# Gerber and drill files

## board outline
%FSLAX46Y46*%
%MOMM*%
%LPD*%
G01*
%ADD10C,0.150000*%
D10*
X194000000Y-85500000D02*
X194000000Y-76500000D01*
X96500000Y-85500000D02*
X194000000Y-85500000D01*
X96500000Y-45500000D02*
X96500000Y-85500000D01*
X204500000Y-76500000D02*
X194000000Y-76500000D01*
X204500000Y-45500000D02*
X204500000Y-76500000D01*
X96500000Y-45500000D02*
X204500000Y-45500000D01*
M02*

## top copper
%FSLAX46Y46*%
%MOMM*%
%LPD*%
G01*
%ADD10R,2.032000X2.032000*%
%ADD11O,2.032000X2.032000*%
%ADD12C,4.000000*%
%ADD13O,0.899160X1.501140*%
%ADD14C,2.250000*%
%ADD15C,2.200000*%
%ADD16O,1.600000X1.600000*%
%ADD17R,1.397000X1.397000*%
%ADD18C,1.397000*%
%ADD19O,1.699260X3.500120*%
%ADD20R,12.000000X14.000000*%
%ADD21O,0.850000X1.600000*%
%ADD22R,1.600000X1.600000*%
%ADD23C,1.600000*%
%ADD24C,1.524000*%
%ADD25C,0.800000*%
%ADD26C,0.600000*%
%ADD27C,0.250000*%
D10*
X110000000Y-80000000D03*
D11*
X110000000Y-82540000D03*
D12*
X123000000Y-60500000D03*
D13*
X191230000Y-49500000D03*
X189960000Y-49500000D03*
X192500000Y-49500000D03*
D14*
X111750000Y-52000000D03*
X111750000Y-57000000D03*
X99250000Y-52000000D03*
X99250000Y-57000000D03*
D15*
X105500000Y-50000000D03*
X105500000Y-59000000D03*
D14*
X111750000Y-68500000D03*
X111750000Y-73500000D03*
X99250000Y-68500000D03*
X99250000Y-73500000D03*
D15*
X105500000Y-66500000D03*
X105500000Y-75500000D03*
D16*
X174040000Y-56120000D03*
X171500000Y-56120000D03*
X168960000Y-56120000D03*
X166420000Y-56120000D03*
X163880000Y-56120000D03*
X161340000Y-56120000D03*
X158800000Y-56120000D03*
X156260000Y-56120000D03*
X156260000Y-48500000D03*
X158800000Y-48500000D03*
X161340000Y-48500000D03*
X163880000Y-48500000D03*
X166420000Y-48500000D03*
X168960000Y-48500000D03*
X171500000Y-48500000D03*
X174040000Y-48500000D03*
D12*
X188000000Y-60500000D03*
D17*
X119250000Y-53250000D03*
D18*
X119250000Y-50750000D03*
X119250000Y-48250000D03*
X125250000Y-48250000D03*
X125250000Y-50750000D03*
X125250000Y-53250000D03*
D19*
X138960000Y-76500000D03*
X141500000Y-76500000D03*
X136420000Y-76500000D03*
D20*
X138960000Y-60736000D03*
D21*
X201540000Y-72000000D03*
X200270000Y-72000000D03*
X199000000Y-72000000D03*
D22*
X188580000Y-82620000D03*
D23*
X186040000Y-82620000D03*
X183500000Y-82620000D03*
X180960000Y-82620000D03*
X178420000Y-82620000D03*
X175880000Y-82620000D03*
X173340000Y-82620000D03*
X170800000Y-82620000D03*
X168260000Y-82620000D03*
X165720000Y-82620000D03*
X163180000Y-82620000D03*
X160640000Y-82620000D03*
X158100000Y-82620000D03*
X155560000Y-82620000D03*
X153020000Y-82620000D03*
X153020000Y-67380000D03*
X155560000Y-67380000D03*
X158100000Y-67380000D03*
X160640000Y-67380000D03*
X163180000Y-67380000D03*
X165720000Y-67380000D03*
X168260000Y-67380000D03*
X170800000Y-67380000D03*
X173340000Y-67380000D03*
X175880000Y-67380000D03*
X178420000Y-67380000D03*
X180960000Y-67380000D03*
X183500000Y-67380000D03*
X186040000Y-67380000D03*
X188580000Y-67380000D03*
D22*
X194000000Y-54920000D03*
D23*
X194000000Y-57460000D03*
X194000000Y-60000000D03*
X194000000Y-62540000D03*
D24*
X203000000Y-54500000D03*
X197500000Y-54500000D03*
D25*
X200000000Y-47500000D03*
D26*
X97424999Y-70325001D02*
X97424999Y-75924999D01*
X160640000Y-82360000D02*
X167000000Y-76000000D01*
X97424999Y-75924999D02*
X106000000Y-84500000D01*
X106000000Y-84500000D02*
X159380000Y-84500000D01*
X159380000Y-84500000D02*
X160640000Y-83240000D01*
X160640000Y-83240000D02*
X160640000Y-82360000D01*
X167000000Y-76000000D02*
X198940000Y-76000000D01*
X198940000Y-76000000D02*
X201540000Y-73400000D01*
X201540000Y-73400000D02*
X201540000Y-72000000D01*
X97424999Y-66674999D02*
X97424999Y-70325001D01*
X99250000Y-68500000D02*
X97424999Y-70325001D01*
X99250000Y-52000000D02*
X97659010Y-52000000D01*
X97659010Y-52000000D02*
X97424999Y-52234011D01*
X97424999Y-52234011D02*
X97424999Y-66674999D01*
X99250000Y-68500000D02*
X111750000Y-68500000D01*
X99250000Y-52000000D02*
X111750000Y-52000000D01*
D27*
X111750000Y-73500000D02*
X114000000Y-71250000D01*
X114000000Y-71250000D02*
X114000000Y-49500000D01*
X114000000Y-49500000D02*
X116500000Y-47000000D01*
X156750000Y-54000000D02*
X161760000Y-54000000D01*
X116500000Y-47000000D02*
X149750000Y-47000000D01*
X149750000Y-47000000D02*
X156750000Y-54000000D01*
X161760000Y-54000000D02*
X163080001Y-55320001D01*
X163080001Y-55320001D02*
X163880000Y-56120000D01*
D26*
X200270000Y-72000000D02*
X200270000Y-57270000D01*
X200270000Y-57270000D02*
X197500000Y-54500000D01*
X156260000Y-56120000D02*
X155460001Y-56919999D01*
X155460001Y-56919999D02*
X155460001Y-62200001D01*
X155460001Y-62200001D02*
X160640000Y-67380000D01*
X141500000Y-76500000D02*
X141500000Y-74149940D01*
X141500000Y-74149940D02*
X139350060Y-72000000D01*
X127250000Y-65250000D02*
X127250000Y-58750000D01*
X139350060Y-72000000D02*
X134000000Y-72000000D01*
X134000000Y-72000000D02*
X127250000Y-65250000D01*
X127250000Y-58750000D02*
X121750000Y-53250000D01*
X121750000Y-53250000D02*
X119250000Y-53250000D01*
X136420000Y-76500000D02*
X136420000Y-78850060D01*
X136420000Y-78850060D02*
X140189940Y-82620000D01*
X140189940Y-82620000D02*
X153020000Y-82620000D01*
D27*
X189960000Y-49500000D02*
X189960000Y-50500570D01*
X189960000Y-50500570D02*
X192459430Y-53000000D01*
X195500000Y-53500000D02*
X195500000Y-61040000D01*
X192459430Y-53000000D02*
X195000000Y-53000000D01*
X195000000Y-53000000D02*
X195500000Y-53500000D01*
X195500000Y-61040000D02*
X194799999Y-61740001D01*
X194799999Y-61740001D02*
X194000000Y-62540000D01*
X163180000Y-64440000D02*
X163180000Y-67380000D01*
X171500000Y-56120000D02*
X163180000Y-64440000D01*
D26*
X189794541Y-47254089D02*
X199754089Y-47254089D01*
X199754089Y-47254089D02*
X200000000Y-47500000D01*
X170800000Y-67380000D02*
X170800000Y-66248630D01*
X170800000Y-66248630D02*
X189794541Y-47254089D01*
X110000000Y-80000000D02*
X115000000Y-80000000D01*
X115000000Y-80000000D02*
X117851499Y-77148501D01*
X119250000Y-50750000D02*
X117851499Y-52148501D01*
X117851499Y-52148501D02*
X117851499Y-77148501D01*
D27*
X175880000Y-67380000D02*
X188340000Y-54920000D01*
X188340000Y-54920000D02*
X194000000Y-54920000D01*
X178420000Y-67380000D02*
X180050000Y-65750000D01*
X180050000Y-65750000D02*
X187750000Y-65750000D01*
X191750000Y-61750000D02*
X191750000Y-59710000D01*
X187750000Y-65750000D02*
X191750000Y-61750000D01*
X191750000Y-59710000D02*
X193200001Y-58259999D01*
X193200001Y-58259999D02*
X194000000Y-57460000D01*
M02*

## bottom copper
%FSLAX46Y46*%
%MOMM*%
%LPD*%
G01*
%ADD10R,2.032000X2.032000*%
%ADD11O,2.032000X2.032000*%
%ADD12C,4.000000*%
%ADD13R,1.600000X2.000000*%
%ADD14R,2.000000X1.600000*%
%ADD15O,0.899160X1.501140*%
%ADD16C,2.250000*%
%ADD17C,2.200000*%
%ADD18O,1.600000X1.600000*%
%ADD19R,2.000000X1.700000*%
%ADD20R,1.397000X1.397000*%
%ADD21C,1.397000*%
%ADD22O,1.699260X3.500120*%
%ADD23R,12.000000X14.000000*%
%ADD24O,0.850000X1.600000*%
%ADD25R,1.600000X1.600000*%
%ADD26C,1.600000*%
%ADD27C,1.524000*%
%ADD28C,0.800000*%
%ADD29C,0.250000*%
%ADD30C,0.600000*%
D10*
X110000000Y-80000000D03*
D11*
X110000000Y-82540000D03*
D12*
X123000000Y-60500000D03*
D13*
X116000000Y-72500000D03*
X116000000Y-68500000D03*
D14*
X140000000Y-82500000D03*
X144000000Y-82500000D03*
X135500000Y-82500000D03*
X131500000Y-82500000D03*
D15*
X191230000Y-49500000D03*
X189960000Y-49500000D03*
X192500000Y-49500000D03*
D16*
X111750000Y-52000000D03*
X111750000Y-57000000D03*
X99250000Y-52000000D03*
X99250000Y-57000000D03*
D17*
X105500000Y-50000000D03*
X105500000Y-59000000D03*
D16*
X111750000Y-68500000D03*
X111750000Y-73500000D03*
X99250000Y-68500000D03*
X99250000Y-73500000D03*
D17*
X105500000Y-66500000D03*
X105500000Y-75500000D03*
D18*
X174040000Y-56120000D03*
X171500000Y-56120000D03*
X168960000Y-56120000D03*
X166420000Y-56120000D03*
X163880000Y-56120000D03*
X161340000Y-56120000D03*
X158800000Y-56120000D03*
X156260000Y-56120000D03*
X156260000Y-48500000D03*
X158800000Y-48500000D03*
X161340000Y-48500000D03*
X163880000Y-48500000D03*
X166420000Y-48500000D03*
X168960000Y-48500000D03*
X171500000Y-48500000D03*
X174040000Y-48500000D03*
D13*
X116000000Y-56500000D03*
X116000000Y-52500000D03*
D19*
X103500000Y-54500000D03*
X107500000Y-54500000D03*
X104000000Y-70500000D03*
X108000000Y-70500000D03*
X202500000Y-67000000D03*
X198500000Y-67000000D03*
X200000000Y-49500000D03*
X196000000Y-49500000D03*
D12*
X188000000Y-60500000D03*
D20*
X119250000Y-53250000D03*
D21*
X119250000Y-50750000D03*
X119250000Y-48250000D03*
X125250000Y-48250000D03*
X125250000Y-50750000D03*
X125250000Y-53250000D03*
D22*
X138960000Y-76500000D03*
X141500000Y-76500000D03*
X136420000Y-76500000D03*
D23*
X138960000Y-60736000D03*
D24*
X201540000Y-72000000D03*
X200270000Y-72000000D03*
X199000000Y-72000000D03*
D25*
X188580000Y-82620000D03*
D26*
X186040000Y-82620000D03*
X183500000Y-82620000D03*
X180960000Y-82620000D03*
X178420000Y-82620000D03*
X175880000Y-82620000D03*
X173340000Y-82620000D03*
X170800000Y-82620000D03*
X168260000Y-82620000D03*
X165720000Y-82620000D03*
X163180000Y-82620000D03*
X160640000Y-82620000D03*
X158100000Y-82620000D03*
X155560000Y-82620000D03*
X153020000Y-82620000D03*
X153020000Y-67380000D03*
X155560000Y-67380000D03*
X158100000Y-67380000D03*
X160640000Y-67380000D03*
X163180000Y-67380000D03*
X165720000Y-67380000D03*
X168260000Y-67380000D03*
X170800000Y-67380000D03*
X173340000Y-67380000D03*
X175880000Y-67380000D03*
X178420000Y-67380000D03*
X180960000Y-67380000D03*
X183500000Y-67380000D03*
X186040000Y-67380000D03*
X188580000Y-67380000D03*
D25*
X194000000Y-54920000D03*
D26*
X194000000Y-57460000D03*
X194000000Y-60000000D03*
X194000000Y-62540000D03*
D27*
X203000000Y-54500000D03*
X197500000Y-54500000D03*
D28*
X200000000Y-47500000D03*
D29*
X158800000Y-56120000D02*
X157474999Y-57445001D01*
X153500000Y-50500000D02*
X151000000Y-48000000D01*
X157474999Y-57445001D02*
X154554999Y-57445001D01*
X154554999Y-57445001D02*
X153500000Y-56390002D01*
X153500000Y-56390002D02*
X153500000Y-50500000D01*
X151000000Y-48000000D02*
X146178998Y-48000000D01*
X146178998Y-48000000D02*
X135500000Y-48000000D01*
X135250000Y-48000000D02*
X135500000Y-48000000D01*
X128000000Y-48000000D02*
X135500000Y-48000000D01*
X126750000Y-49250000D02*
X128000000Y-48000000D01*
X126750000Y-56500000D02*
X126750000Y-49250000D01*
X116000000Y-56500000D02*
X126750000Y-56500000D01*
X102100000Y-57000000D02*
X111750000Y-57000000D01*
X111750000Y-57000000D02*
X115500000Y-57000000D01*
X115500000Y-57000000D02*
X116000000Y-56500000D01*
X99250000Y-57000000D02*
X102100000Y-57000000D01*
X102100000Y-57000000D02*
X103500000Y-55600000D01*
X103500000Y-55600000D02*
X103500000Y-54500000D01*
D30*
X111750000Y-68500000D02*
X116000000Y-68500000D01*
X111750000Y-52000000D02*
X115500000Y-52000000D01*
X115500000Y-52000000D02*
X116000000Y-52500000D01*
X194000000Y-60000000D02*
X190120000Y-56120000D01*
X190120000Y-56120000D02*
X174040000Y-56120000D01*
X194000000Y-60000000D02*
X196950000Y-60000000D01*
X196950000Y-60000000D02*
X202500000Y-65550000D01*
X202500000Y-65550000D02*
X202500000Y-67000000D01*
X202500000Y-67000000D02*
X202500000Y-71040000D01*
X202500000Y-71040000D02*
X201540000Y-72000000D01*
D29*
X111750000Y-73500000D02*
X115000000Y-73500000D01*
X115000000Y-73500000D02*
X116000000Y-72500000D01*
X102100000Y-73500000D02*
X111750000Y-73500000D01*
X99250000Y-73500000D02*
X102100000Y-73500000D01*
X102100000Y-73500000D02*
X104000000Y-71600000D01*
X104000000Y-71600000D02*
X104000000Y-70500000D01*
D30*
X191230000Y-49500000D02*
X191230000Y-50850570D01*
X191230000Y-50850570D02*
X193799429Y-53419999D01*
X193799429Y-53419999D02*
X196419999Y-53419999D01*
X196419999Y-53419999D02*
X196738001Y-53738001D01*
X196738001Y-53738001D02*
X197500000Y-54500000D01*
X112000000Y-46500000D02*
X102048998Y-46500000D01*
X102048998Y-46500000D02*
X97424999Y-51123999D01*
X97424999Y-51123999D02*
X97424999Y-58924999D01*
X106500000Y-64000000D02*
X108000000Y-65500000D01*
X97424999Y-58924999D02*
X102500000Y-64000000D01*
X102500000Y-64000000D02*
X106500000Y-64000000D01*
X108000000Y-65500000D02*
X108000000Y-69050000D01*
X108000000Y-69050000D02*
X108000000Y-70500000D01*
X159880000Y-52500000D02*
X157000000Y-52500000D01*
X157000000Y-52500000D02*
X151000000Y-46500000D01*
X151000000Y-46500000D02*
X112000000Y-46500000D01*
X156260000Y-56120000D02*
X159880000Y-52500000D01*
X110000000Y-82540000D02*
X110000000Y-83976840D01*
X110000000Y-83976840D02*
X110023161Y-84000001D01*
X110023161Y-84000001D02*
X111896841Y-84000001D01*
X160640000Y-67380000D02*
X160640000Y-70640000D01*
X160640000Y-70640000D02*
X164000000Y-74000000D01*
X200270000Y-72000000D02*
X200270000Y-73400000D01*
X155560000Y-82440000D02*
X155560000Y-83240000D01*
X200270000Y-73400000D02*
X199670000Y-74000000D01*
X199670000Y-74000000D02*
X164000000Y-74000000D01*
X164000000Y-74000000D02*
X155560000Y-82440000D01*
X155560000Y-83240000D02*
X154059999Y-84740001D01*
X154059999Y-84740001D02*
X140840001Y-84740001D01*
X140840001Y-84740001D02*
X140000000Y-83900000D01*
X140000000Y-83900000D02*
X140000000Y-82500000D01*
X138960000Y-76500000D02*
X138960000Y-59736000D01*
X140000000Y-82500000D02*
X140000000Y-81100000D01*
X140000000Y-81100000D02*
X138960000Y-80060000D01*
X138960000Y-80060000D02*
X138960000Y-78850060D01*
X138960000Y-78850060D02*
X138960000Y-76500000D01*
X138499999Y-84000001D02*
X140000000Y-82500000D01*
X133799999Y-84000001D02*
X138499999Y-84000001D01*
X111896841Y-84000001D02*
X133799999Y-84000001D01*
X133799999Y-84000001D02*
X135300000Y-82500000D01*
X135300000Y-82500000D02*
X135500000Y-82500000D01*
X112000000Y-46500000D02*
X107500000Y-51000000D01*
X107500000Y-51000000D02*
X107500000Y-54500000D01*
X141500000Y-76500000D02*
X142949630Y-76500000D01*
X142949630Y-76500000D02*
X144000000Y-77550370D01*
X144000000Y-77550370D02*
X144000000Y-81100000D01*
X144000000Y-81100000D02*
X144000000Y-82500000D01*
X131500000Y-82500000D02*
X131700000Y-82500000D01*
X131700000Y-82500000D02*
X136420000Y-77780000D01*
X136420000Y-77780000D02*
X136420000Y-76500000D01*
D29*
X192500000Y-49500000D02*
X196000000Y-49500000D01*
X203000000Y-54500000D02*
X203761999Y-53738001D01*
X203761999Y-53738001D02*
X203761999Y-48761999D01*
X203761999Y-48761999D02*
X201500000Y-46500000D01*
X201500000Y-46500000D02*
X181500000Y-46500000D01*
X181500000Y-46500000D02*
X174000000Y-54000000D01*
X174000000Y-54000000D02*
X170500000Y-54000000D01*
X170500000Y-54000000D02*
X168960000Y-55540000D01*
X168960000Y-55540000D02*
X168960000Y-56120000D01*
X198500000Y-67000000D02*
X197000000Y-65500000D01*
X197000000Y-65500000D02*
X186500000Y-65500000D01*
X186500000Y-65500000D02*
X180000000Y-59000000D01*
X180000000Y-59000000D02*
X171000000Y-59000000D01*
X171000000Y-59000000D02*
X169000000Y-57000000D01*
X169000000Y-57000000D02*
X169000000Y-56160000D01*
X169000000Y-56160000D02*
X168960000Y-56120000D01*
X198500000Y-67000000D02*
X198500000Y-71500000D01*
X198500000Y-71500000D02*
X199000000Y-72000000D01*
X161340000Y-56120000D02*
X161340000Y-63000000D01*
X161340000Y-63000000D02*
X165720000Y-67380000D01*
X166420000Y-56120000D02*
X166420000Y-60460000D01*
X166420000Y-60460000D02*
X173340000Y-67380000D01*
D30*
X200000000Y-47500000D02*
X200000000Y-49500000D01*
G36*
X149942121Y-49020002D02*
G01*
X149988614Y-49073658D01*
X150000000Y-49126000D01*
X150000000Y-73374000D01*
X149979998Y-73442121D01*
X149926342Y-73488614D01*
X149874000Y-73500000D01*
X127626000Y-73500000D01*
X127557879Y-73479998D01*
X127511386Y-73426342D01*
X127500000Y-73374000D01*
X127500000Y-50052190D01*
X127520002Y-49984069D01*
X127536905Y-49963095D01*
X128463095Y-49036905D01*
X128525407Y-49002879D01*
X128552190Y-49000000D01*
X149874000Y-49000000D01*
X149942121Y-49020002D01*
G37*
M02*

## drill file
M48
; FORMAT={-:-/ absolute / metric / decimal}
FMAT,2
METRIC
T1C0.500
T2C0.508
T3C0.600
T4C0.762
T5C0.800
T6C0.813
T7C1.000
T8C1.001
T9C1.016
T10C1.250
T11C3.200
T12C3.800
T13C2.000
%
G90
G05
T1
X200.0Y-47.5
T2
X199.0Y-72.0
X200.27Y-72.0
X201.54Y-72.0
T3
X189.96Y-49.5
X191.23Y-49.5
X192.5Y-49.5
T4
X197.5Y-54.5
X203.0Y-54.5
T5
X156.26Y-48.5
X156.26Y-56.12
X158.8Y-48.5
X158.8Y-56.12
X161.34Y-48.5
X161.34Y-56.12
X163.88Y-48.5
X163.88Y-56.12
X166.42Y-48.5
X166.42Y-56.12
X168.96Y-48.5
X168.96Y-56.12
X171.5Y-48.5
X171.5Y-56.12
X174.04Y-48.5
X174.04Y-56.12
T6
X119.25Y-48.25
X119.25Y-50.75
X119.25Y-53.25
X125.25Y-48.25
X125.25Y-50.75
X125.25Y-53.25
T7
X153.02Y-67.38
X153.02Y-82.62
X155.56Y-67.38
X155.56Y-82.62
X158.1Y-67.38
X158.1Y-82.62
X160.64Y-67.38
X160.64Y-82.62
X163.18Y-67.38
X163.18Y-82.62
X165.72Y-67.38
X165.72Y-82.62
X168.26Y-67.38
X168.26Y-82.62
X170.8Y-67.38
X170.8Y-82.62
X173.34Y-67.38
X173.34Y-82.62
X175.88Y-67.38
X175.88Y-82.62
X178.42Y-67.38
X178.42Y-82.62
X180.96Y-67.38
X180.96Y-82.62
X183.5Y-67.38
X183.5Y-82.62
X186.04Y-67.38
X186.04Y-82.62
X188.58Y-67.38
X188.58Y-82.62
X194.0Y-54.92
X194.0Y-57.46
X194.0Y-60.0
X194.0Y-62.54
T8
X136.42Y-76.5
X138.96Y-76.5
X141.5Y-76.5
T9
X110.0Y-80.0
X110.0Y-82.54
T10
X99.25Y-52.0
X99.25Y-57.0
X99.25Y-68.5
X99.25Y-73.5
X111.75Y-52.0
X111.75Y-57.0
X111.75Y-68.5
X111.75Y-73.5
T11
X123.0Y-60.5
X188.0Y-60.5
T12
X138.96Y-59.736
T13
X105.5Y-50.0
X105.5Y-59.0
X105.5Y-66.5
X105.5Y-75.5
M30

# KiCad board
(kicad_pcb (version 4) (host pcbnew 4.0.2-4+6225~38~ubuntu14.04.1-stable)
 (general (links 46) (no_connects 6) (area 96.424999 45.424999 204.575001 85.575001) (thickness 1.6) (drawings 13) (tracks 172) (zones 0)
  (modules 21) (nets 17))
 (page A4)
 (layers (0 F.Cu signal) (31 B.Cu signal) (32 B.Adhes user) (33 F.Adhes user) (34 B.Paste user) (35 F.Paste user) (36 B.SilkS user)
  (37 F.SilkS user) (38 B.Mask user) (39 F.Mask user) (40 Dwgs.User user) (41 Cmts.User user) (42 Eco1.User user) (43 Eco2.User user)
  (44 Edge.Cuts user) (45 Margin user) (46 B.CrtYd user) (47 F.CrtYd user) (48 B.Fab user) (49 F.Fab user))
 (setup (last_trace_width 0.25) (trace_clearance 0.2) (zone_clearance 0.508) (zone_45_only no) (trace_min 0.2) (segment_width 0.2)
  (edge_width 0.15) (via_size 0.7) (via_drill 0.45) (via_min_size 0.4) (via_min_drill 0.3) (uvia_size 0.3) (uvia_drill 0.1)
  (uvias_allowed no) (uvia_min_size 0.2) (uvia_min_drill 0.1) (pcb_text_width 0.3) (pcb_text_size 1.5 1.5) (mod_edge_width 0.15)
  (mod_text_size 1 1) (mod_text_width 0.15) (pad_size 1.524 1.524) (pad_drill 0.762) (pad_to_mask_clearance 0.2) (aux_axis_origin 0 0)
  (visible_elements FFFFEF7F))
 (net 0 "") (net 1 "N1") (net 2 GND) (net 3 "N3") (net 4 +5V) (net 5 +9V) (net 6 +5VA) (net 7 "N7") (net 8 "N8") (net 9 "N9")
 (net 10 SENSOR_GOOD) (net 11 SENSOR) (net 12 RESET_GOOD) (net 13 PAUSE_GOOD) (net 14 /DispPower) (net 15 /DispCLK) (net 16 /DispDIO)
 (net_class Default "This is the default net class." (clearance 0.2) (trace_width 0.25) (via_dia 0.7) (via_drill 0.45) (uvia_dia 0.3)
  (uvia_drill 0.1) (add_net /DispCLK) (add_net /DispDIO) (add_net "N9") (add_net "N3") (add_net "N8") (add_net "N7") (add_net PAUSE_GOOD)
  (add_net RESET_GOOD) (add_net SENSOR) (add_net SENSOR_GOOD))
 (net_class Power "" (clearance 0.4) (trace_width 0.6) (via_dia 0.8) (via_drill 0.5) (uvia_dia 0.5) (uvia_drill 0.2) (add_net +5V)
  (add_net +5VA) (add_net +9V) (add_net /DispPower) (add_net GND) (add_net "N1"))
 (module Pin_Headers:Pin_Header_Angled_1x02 (layer B.Cu) (at 110 80 180)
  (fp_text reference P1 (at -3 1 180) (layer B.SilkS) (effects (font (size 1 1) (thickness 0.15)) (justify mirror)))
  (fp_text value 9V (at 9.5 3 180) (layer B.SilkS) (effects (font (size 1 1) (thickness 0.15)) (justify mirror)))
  (pad 1 thru_hole rect (at 0 0 180) (size 2.032 2.032) (drill 1.016) (layers *.Cu *.Mask B.SilkS) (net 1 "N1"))
  (pad 2 thru_hole oval (at 0 -2.54 180) (size 2.032 2.032) (drill 1.016) (layers *.Cu *.Mask B.SilkS) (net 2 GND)))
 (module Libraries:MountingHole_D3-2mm (layer F.Cu) (at 123 60.5)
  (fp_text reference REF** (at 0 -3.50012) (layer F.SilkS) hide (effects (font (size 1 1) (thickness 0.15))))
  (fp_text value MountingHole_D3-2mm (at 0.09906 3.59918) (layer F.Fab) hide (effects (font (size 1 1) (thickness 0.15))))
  (pad 1 thru_hole circle (at 0 0) (size 4 4) (drill 3.2) (layers *.Cu)))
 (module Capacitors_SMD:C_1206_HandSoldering (layer B.Cu) (at 116 70.5 90)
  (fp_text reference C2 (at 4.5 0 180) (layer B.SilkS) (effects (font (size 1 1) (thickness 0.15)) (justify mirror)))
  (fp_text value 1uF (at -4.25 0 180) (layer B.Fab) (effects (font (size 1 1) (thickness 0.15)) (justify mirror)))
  (pad 1 smd rect (at -2 0 90) (size 2 1.6) (layers B.Cu B.Paste B.Mask) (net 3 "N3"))
  (pad 2 smd rect (at 2 0 90) (size 2 1.6) (layers B.Cu B.Paste B.Mask) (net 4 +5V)))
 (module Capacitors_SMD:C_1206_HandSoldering (layer B.Cu) (at 142 82.5)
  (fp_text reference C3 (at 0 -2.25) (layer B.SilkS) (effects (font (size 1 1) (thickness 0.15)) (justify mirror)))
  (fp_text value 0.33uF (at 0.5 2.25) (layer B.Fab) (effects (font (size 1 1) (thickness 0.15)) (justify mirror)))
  (pad 1 smd rect (at -2 0) (size 2 1.6) (layers B.Cu B.Paste B.Mask) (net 2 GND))
  (pad 2 smd rect (at 2 0) (size 2 1.6) (layers B.Cu B.Paste B.Mask) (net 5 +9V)))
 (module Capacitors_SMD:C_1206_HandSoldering (layer B.Cu) (at 133.5 82.5 180)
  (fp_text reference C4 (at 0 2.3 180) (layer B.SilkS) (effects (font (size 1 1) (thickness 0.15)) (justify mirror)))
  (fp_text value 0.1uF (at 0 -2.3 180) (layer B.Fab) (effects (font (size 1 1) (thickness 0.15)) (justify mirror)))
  (pad 1 smd rect (at -2 0 180) (size 2 1.6) (layers B.Cu B.Paste B.Mask) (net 2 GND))
  (pad 2 smd rect (at 2 0 180) (size 2 1.6) (layers B.Cu B.Paste B.Mask) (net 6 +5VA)))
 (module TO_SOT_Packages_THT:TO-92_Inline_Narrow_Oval (layer B.Cu) (at 192.5 49.5 180)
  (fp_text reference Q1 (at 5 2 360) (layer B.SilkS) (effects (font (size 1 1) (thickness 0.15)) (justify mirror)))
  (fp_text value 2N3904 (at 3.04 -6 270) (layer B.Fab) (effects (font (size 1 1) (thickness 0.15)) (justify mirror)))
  (pad 2 thru_hole oval (at 1.27 0) (size 0.89916 1.50114) (drill 0.6) (layers *.Cu *.Mask B.SilkS) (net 2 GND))
  (pad 3 thru_hole oval (at 2.54 0) (size 0.89916 1.50114) (drill 0.6) (layers *.Cu *.Mask B.SilkS) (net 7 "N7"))
  (pad 1 thru_hole oval (at 0 0) (size 0.89916 1.50114) (drill 0.6) (layers *.Cu *.Mask B.SilkS) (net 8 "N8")))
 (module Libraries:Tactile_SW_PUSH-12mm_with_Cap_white (layer F.Cu) (at 105.5 54.5)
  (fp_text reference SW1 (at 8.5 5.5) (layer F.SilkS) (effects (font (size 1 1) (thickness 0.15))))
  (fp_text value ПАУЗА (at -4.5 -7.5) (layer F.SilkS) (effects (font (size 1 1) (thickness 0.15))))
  (pad 1 thru_hole circle (at 6.25 -2.5) (size 2.25 2.25) (drill 1.25) (layers *.Cu *.Mask F.SilkS) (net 4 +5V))
  (pad 2 thru_hole circle (at 6.25 2.5) (size 2.25 2.25) (drill 1.25) (layers *.Cu *.Mask F.SilkS) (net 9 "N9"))
  (pad 1 thru_hole circle (at -6.25 -2.5) (size 2.25 2.25) (drill 1.25) (layers *.Cu *.Mask F.SilkS) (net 4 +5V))
  (pad 2 thru_hole circle (at -6.25 2.5) (size 2.25 2.25) (drill 1.25) (layers *.Cu *.Mask F.SilkS) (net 9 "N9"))
  (pad "" np_thru_hole circle (at 0 -4.5) (size 2.2 2.2) (drill 2) (layers *.Cu *.Mask F.SilkS))
  (pad "" np_thru_hole circle (at 0 4.5) (size 2.2 2.2) (drill 2) (layers *.Cu *.Mask F.SilkS)))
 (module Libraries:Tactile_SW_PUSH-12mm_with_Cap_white (layer F.Cu) (at 105.5 71)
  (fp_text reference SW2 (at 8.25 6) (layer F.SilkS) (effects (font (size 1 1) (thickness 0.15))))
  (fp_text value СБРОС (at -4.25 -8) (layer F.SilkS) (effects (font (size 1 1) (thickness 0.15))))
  (pad 1 thru_hole circle (at 6.25 -2.5) (size 2.25 2.25) (drill 1.25) (layers *.Cu *.Mask F.SilkS) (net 4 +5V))
  (pad 2 thru_hole circle (at 6.25 2.5) (size 2.25 2.25) (drill 1.25) (layers *.Cu *.Mask F.SilkS) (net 3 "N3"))
  (pad 1 thru_hole circle (at -6.25 -2.5) (size 2.25 2.25) (drill 1.25) (layers *.Cu *.Mask F.SilkS) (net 4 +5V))
  (pad 2 thru_hole circle (at -6.25 2.5) (size 2.25 2.25) (drill 1.25) (layers *.Cu *.Mask F.SilkS) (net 3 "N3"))
  (pad "" np_thru_hole circle (at 0 -4.5) (size 2.2 2.2) (drill 2) (layers *.Cu *.Mask F.SilkS))
  (pad "" np_thru_hole circle (at 0 4.5) (size 2.2 2.2) (drill 2) (layers *.Cu *.Mask F.SilkS)))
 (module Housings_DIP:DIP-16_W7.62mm (layer B.Cu) (at 174.04 56.12 90)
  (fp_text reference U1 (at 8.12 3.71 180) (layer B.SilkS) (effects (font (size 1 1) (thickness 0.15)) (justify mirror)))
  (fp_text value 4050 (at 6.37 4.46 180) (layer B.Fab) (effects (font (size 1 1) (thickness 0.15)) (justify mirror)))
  (pad 1 thru_hole oval (at 0 0 90) (size 1.6 1.6) (drill 0.8) (layers *.Cu *.Mask B.SilkS) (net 4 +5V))
  (pad 2 thru_hole oval (at 0 -2.54 90) (size 1.6 1.6) (drill 0.8) (layers *.Cu *.Mask B.SilkS) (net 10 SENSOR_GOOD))
  (pad 3 thru_hole oval (at 0 -5.08 90) (size 1.6 1.6) (drill 0.8) (layers *.Cu *.Mask B.SilkS) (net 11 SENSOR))
  (pad 4 thru_hole oval (at 0 -7.62 90) (size 1.6 1.6) (drill 0.8) (layers *.Cu *.Mask B.SilkS) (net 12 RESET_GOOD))
  (pad 5 thru_hole oval (at 0 -10.16 90) (size 1.6 1.6) (drill 0.8) (layers *.Cu *.Mask B.SilkS) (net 3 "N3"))
  (pad 6 thru_hole oval (at 0 -12.7 90) (size 1.6 1.6) (drill 0.8) (layers *.Cu *.Mask B.SilkS) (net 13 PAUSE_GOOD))
  (pad 7 thru_hole oval (at 0 -15.24 90) (size 1.6 1.6) (drill 0.8) (layers *.Cu *.Mask B.SilkS) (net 9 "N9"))
  (pad 8 thru_hole oval (at 0 -17.78 90) (size 1.6 1.6) (drill 0.8) (layers *.Cu *.Mask B.SilkS) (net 2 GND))
  (pad 9 thru_hole oval (at 7.62 -17.78 90) (size 1.6 1.6) (drill 0.8) (layers *.Cu *.Mask B.SilkS))
  (pad 10 thru_hole oval (at 7.62 -15.24 90) (size 1.6 1.6) (drill 0.8) (layers *.Cu *.Mask B.SilkS))
  (pad 11 thru_hole oval (at 7.62 -12.7 90) (size 1.6 1.6) (drill 0.8) (layers *.Cu *.Mask B.SilkS))
  (pad 12 thru_hole oval (at 7.62 -10.16 90) (size 1.6 1.6) (drill 0.8) (layers *.Cu *.Mask B.SilkS))
  (pad 13 thru_hole oval (at 7.62 -7.62 90) (size 1.6 1.6) (drill 0.8) (layers *.Cu *.Mask B.SilkS))
  (pad 14 thru_hole oval (at 7.62 -5.08 90) (size 1.6 1.6) (drill 0.8) (layers *.Cu *.Mask B.SilkS))
  (pad 15 thru_hole oval (at 7.62 -2.54 90) (size 1.6 1.6) (drill 0.8) (layers *.Cu *.Mask B.SilkS))
  (pad 16 thru_hole oval (at 7.62 0 90) (size 1.6 1.6) (drill 0.8) (layers *.Cu *.Mask B.SilkS)))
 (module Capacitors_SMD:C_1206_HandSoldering (layer B.Cu) (at 116 54.5 90)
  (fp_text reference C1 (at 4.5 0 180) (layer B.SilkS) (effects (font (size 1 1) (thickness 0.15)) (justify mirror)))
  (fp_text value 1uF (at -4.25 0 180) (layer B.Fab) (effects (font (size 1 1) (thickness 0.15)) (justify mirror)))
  (pad 1 smd rect (at -2 0 90) (size 2 1.6) (layers B.Cu B.Paste B.Mask) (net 9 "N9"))
  (pad 2 smd rect (at 2 0 90) (size 2 1.6) (layers B.Cu B.Paste B.Mask) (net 4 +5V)))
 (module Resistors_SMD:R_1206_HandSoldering (layer B.Cu) (at 105.5 54.5)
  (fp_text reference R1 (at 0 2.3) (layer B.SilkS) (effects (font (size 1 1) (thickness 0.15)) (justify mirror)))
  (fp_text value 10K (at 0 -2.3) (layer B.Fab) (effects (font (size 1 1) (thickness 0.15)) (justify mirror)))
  (pad 1 smd rect (at -2 0) (size 2 1.7) (layers B.Cu B.Paste B.Mask) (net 9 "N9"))
  (pad 2 smd rect (at 2 0) (size 2 1.7) (layers B.Cu B.Paste B.Mask) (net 2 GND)))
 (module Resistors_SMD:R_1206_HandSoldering (layer B.Cu) (at 106 70.5)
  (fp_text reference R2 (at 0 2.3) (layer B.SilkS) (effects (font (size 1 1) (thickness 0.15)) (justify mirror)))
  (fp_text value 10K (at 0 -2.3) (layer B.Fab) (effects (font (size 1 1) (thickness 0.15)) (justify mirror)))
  (pad 1 smd rect (at -2 0) (size 2 1.7) (layers B.Cu B.Paste B.Mask) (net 3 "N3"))
  (pad 2 smd rect (at 2 0) (size 2 1.7) (layers B.Cu B.Paste B.Mask) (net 2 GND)))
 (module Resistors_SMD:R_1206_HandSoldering (layer B.Cu) (at 200.5 67 180)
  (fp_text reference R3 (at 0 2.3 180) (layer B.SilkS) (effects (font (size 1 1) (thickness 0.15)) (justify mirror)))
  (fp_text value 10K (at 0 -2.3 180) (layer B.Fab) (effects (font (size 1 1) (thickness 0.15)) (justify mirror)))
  (pad 1 smd rect (at -2 0 180) (size 2 1.7) (layers B.Cu B.Paste B.Mask) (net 4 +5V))
  (pad 2 smd rect (at 2 0 180) (size 2 1.7) (layers B.Cu B.Paste B.Mask) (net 11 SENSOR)))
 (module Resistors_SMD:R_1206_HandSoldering (layer B.Cu) (at 198 49.5 180)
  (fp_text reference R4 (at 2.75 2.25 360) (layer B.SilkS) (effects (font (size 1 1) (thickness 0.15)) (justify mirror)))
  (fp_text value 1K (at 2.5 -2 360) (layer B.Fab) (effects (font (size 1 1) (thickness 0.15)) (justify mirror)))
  (pad 1 smd rect (at -2 0 180) (size 2 1.7) (layers B.Cu B.Paste B.Mask) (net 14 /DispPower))
  (pad 2 smd rect (at 2 0 180) (size 2 1.7) (layers B.Cu B.Paste B.Mask) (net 8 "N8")))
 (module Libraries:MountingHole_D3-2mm (layer F.Cu) (at 188 60.5)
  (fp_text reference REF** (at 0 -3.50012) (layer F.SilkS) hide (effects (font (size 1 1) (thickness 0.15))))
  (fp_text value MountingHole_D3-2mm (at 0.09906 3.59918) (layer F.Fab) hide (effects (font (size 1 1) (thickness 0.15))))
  (pad 1 thru_hole circle (at 0 0) (size 4 4) (drill 3.2) (layers *.Cu)))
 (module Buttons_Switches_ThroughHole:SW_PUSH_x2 (layer B.Cu) (at 119.25 53.25 90)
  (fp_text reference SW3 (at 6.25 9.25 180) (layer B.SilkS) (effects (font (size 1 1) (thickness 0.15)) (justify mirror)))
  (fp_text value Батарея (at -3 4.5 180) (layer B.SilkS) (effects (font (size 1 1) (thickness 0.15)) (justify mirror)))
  (pad 1 thru_hole rect (at 0 0 90) (size 1.397 1.397) (drill 0.8128) (layers *.Cu *.Mask B.SilkS) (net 5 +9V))
  (pad 2 thru_hole circle (at 2.5 0 90) (size 1.397 1.397) (drill 0.8128) (layers *.Cu *.Mask B.SilkS) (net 1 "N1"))
  (pad 3 thru_hole circle (at 5 0 90) (size 1.397 1.397) (drill 0.8128) (layers *.Cu *.Mask B.SilkS))
  (pad 4 thru_hole circle (at 5 6 90) (size 1.397 1.397) (drill 0.8128) (layers *.Cu *.Mask B.SilkS))
  (pad 5 thru_hole circle (at 2.5 6 90) (size 1.397 1.397) (drill 0.8128) (layers *.Cu *.Mask B.SilkS))
  (pad 6 thru_hole circle (at 0 6 90) (size 1.397 1.397) (drill 0.8128) (layers *.Cu *.Mask B.SilkS)))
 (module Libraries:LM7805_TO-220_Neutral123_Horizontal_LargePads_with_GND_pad (layer B.Cu) (at 138.96 76.5 180)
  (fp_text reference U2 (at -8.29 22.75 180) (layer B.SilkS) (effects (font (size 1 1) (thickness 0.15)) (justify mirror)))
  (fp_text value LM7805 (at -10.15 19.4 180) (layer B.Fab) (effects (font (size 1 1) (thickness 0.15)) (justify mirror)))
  (pad 2 thru_hole oval (at 0 0 90) (size 3.50012 1.69926) (drill 1.00076) (layers *.Cu *.Mask B.SilkS) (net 2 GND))
  (pad 1 thru_hole oval (at -2.54 0 90) (size 3.50012 1.69926) (drill 1.00076) (layers *.Cu *.Mask B.SilkS) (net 5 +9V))
  (pad 3 thru_hole oval (at 2.54 0 90) (size 3.50012 1.69926) (drill 1.00076) (layers *.Cu *.Mask B.SilkS) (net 6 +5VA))
  (pad 2 thru_hole rect (at 0 16.764 90) (size 14 12) (drill 3.79984 (offset -1 0)) (layers B.Cu B.SilkS B.Mask) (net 2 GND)))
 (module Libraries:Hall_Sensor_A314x (layer F.Cu) (at 200.27 72 180)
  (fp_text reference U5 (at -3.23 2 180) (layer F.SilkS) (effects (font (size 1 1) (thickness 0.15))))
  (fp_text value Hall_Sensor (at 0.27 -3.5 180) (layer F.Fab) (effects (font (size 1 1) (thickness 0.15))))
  (pad 1 thru_hole oval (at -1.27 0 180) (size 0.85 1.6) (drill 0.508) (layers *.Cu *.Mask F.SilkS) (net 4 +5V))
  (pad 2 thru_hole oval (at 0 0 180) (size 0.85 1.6) (drill 0.508) (layers *.Cu *.Mask F.SilkS) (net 2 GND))
  (pad 3 thru_hole oval (at 1.27 0 180) (size 0.85 1.6) (drill 0.508) (layers *.Cu *.Mask F.SilkS) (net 11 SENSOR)))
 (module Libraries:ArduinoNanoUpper (layer B.Cu) (at 170.8 75 180)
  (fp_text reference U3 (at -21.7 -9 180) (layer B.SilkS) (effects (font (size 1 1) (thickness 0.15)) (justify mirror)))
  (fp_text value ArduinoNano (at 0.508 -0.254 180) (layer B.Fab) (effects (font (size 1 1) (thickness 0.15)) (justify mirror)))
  (pad 1 thru_hole rect (at -17.78 -7.62 180) (size 1.6 1.6) (drill 1) (layers *.Cu *.Mask B.SilkS))
  (pad 2 thru_hole circle (at -15.24 -7.62 180) (size 1.6 1.6) (drill 1) (layers *.Cu *.Mask B.SilkS))
  (pad 3 thru_hole circle (at -12.7 -7.62 180) (size 1.6 1.6) (drill 1) (layers *.Cu *.Mask B.SilkS))
  (pad 4 thru_hole circle (at -10.16 -7.62 180) (size 1.6 1.6) (drill 1) (layers *.Cu *.Mask B.SilkS))
  (pad 5 thru_hole circle (at -7.62 -7.62 180) (size 1.6 1.6) (drill 1) (layers *.Cu *.Mask B.SilkS))
  (pad 6 thru_hole circle (at -5.08 -7.62 180) (size 1.6 1.6) (drill 1) (layers *.Cu *.Mask B.SilkS))
  (pad 7 thru_hole circle (at -2.54 -7.62 180) (size 1.6 1.6) (drill 1) (layers *.Cu *.Mask B.SilkS))
  (pad 8 thru_hole circle (at 0 -7.62 180) (size 1.6 1.6) (drill 1) (layers *.Cu *.Mask B.SilkS))
  (pad 9 thru_hole circle (at 2.54 -7.62 180) (size 1.6 1.6) (drill 1) (layers *.Cu *.Mask B.SilkS))
  (pad 10 thru_hole circle (at 5.08 -7.62 180) (size 1.6 1.6) (drill 1) (layers *.Cu *.Mask B.SilkS))
  (pad 11 thru_hole circle (at 7.62 -7.62 180) (size 1.6 1.6) (drill 1) (layers *.Cu *.Mask B.SilkS))
  (pad 12 thru_hole circle (at 10.16 -7.62 180) (size 1.6 1.6) (drill 1) (layers *.Cu *.Mask B.SilkS) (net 4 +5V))
  (pad 13 thru_hole circle (at 12.7 -7.62 180) (size 1.6 1.6) (drill 1) (layers *.Cu *.Mask B.SilkS))
  (pad 14 thru_hole circle (at 15.24 -7.62 180) (size 1.6 1.6) (drill 1) (layers *.Cu *.Mask B.SilkS) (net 2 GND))
  (pad 15 thru_hole circle (at 17.78 -7.62 180) (size 1.6 1.6) (drill 1) (layers *.Cu *.Mask B.SilkS) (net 6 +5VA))
  (pad 16 thru_hole circle (at 17.78 7.62 180) (size 1.6 1.6) (drill 1) (layers *.Cu *.Mask B.SilkS))
  (pad 17 thru_hole circle (at 15.24 7.62 180) (size 1.6 1.6) (drill 1) (layers *.Cu *.Mask B.SilkS))
  (pad 18 thru_hole circle (at 12.7 7.62 180) (size 1.6 1.6) (drill 1) (layers *.Cu *.Mask B.SilkS))
  (pad 19 thru_hole circle (at 10.16 7.62 180) (size 1.6 1.6) (drill 1) (layers *.Cu *.Mask B.SilkS) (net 2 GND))
  (pad 20 thru_hole circle (at 7.62 7.62 180) (size 1.6 1.6) (drill 1) (layers *.Cu *.Mask B.SilkS) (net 10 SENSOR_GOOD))
  (pad 21 thru_hole circle (at 5.08 7.62 180) (size 1.6 1.6) (drill 1) (layers *.Cu *.Mask B.SilkS) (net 13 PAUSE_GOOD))
  (pad 22 thru_hole circle (at 2.54 7.62 180) (size 1.6 1.6) (drill 1) (layers *.Cu *.Mask B.SilkS))
  (pad 23 thru_hole circle (at 0 7.62 180) (size 1.6 1.6) (drill 1) (layers *.Cu *.Mask B.SilkS) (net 14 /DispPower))
  (pad 24 thru_hole circle (at -2.54 7.62 180) (size 1.6 1.6) (drill 1) (layers *.Cu *.Mask B.SilkS) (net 12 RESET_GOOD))
  (pad 25 thru_hole circle (at -5.08 7.62 180) (size 1.6 1.6) (drill 1) (layers *.Cu *.Mask B.SilkS) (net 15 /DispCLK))
  (pad 26 thru_hole circle (at -7.62 7.62 180) (size 1.6 1.6) (drill 1) (layers *.Cu *.Mask B.SilkS) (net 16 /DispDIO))
  (pad 27 thru_hole circle (at -10.16 7.62 180) (size 1.6 1.6) (drill 1) (layers *.Cu *.Mask B.SilkS))
  (pad 28 thru_hole circle (at -12.7 7.62 180) (size 1.6 1.6) (drill 1) (layers *.Cu *.Mask B.SilkS))
  (pad 29 thru_hole circle (at -15.24 7.62 180) (size 1.6 1.6) (drill 1) (layers *.Cu *.Mask B.SilkS))
  (pad 30 thru_hole circle (at -17.78 7.62 180) (size 1.6 1.6) (drill 1) (layers *.Cu *.Mask B.SilkS)))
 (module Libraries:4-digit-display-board (layer F.Cu) (at 175.54 58.73)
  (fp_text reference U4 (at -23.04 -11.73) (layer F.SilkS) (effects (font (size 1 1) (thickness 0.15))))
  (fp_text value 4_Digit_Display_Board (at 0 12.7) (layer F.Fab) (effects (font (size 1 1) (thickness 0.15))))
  (pad 1 thru_hole rect (at 18.46 -3.81) (size 1.6 1.6) (drill 1) (layers *.Cu *.Mask F.SilkS) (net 15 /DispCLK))
  (pad 2 thru_hole circle (at 18.46 -1.27) (size 1.6 1.6) (drill 1) (layers *.Cu *.Mask F.SilkS) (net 16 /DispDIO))
  (pad 3 thru_hole circle (at 18.46 1.27) (size 1.6 1.6) (drill 1) (layers *.Cu *.Mask F.SilkS) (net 4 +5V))
  (pad 4 thru_hole circle (at 18.46 3.81) (size 1.6 1.6) (drill 1) (layers *.Cu *.Mask F.SilkS) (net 7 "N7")))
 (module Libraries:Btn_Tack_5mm (layer F.Cu) (at 203 54.5 180)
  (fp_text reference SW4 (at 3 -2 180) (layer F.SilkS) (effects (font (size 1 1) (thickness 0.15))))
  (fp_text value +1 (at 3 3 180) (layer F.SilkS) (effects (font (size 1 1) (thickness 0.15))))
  (pad 1 thru_hole circle (at 0 0 180) (size 1.524 1.524) (drill 0.762) (layers *.Cu *.Mask F.SilkS) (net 11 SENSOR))
  (pad 2 thru_hole circle (at 5.5 0 180) (size 1.524 1.524) (drill 0.762) (layers *.Cu *.Mask F.SilkS) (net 2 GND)))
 (gr_line (start 194 85.5) (end 194 76.5) (layer Edge.Cuts) (width 0.15))
 (gr_line (start 96.5 85.5) (end 194 85.5) (layer Edge.Cuts) (width 0.15))
 (gr_line (start 96.5 45.5) (end 96.5 85.5) (layer Edge.Cuts) (width 0.15))
 (gr_line (start 204.5 76.5) (end 194 76.5) (layer Edge.Cuts) (width 0.15))
 (gr_line (start 204.5 45.5) (end 204.5 76.5) (layer Edge.Cuts) (width 0.15))
 (gr_line (start 96.5 45.5) (end 204.5 45.5) (layer Edge.Cuts) (width 0.15))
 (segment (start 158.8 56.12) (end 157.474999 57.445001) (width 0.25) (layer B.Cu) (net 9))
 (segment (start 153.5 50.5) (end 151 48) (width 0.25) (layer B.Cu) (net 9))
 (segment (start 157.474999 57.445001) (end 154.554999 57.445001) (width 0.25) (layer B.Cu) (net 9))
 (segment (start 154.554999 57.445001) (end 153.5 56.390002) (width 0.25) (layer B.Cu) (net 9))
 (segment (start 153.5 56.390002) (end 153.5 50.5) (width 0.25) (layer B.Cu) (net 9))
 (segment (start 151 48) (end 146.178998 48) (width 0.25) (layer B.Cu) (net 9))
 (segment (start 146.178998 48) (end 135.5 48) (width 0.25) (layer B.Cu) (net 9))
 (segment (start 135.25 48) (end 135.5 48) (width 0.25) (layer B.Cu) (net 9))
 (segment (start 128 48) (end 135.5 48) (width 0.25) (layer B.Cu) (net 9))
 (segment (start 126.75 49.25) (end 128 48) (width 0.25) (layer B.Cu) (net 9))
 (segment (start 126.75 56.5) (end 126.75 49.25) (width 0.25) (layer B.Cu) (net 9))
 (segment (start 116 56.5) (end 126.75 56.5) (width 0.25) (layer B.Cu) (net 9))
 (segment (start 102.1 57) (end 111.75 57) (width 0.25) (layer B.Cu) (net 9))
 (segment (start 111.75 57) (end 115.5 57) (width 0.25) (layer B.Cu) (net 9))
 (segment (start 115.5 57) (end 116 56.5) (width 0.25) (layer B.Cu) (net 9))
 (segment (start 99.25 57) (end 102.1 57) (width 0.25) (layer B.Cu) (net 9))
 (segment (start 102.1 57) (end 103.5 55.6) (width 0.25) (layer B.Cu) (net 9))
 (segment (start 103.5 55.6) (end 103.5 54.5) (width 0.25) (layer B.Cu) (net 9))
 (segment (start 97.424999 70.325001) (end 97.424999 75.924999) (width 0.6) (layer F.Cu) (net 4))
 (segment (start 160.64 82.36) (end 167 76) (width 0.6) (layer F.Cu) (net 4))
 (segment (start 97.424999 75.924999) (end 106 84.5) (width 0.6) (layer F.Cu) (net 4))
 (segment (start 106 84.5) (end 159.38 84.5) (width 0.6) (layer F.Cu) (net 4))
 (segment (start 159.38 84.5) (end 160.64 83.24) (width 0.6) (layer F.Cu) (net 4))
 (segment (start 160.64 83.24) (end 160.64 82.36) (width 0.6) (layer F.Cu) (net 4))
 (segment (start 167 76) (end 198.94 76) (width 0.6) (layer F.Cu) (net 4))
 (segment (start 198.94 76) (end 201.54 73.4) (width 0.6) (layer F.Cu) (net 4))
 (segment (start 201.54 73.4) (end 201.54 72) (width 0.6) (layer F.Cu) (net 4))
 (segment (start 97.424999 66.674999) (end 97.424999 70.325001) (width 0.6) (layer F.Cu) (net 4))
 (segment (start 99.25 68.5) (end 97.424999 70.325001) (width 0.6) (layer F.Cu) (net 4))
 (segment (start 99.25 52) (end 97.65901 52) (width 0.6) (layer F.Cu) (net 4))
 (segment (start 97.65901 52) (end 97.424999 52.234011) (width 0.6) (layer F.Cu) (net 4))
 (segment (start 97.424999 52.234011) (end 97.424999 66.674999) (width 0.6) (layer F.Cu) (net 4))
 (segment (start 99.25 68.5) (end 111.75 68.5) (width 0.6) (layer F.Cu) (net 4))
 (segment (start 99.25 52) (end 111.75 52) (width 0.6) (layer F.Cu) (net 4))
 (segment (start 111.75 68.5) (end 116 68.5) (width 0.6) (layer B.Cu) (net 4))
 (segment (start 111.75 52) (end 115.5 52) (width 0.6) (layer B.Cu) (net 4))
 (segment (start 115.5 52) (end 116 52.5) (width 0.6) (layer B.Cu) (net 4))
 (segment (start 194 60) (end 190.12 56.12) (width 0.6) (layer B.Cu) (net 4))
 (segment (start 190.12 56.12) (end 174.04 56.12) (width 0.6) (layer B.Cu) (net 4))
 (segment (start 194 60) (end 196.95 60) (width 0.6) (layer B.Cu) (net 4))
 (segment (start 196.95 60) (end 202.5 65.55) (width 0.6) (layer B.Cu) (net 4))
 (segment (start 202.5 65.55) (end 202.5 67) (width 0.6) (layer B.Cu) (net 4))
 (segment (start 202.5 67) (end 202.5 71.04) (width 0.6) (layer B.Cu) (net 4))
 (segment (start 202.5 71.04) (end 201.54 72) (width 0.6) (layer B.Cu) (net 4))
 (segment (start 111.75 73.5) (end 114 71.25) (width 0.25) (layer F.Cu) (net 3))
 (segment (start 114 71.25) (end 114 49.5) (width 0.25) (layer F.Cu) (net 3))
 (segment (start 114 49.5) (end 116.5 47) (width 0.25) (layer F.Cu) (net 3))
 (segment (start 156.75 54) (end 161.76 54) (width 0.25) (layer F.Cu) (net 3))
 (segment (start 116.5 47) (end 149.75 47) (width 0.25) (layer F.Cu) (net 3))
 (segment (start 149.75 47) (end 156.75 54) (width 0.25) (layer F.Cu) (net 3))
 (segment (start 161.76 54) (end 163.080001 55.320001) (width 0.25) (layer F.Cu) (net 3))
 (segment (start 163.080001 55.320001) (end 163.88 56.12) (width 0.25) (layer F.Cu) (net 3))
 (segment (start 111.75 73.5) (end 115 73.5) (width 0.25) (layer B.Cu) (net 3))
 (segment (start 115 73.5) (end 116 72.5) (width 0.25) (layer B.Cu) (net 3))
 (segment (start 102.1 73.5) (end 111.75 73.5) (width 0.25) (layer B.Cu) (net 3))
 (segment (start 99.25 73.5) (end 102.1 73.5) (width 0.25) (layer B.Cu) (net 3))
 (segment (start 102.1 73.5) (end 104 71.6) (width 0.25) (layer B.Cu) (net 3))
 (segment (start 104 71.6) (end 104 70.5) (width 0.25) (layer B.Cu) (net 3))
 (segment (start 200.27 72) (end 200.27 57.27) (width 0.6) (layer F.Cu) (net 2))
 (segment (start 200.27 57.27) (end 197.5 54.5) (width 0.6) (layer F.Cu) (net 2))
 (segment (start 191.23 49.5) (end 191.23 50.85057) (width 0.6) (layer B.Cu) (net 2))
 (segment (start 191.23 50.85057) (end 193.799429 53.419999) (width 0.6) (layer B.Cu) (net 2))
 (segment (start 193.799429 53.419999) (end 196.419999 53.419999) (width 0.6) (layer B.Cu) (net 2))
 (segment (start 196.419999 53.419999) (end 196.738001 53.738001) (width 0.6) (layer B.Cu) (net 2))
 (segment (start 196.738001 53.738001) (end 197.5 54.5) (width 0.6) (layer B.Cu) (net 2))
 (segment (start 112 46.5) (end 102.048998 46.5) (width 0.6) (layer B.Cu) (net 2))
 (segment (start 102.048998 46.5) (end 97.424999 51.123999) (width 0.6) (layer B.Cu) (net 2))
 (segment (start 97.424999 51.123999) (end 97.424999 58.924999) (width 0.6) (layer B.Cu) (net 2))
 (segment (start 106.5 64) (end 108 65.5) (width 0.6) (layer B.Cu) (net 2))
 (segment (start 97.424999 58.924999) (end 102.5 64) (width 0.6) (layer B.Cu) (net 2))
 (segment (start 102.5 64) (end 106.5 64) (width 0.6) (layer B.Cu) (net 2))
 (segment (start 108 65.5) (end 108 69.05) (width 0.6) (layer B.Cu) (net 2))
 (segment (start 108 69.05) (end 108 70.5) (width 0.6) (layer B.Cu) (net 2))
 (segment (start 159.88 52.5) (end 157 52.5) (width 0.6) (layer B.Cu) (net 2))
 (segment (start 157 52.5) (end 151 46.5) (width 0.6) (layer B.Cu) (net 2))
 (segment (start 151 46.5) (end 112 46.5) (width 0.6) (layer B.Cu) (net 2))
 (segment (start 156.26 56.12) (end 159.88 52.5) (width 0.6) (layer B.Cu) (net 2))
 (segment (start 110 82.54) (end 110 83.97684) (width 0.6) (layer B.Cu) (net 2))
 (segment (start 110 83.97684) (end 110.023161 84.000001) (width 0.6) (layer B.Cu) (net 2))
 (segment (start 110.023161 84.000001) (end 111.896841 84.000001) (width 0.6) (layer B.Cu) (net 2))
 (segment (start 160.64 67.38) (end 160.64 70.64) (width 0.6) (layer B.Cu) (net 2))
 (segment (start 160.64 70.64) (end 164 74) (width 0.6) (layer B.Cu) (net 2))
 (segment (start 156.26 56.12) (end 155.460001 56.919999) (width 0.6) (layer F.Cu) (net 2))
 (segment (start 155.460001 56.919999) (end 155.460001 62.200001) (width 0.6) (layer F.Cu) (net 2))
 (segment (start 155.460001 62.200001) (end 160.64 67.38) (width 0.6) (layer F.Cu) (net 2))
 (segment (start 200.27 72) (end 200.27 73.4) (width 0.6) (layer B.Cu) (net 2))
 (segment (start 155.56 82.44) (end 155.56 83.24) (width 0.6) (layer B.Cu) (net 2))
 (segment (start 200.27 73.4) (end 199.67 74) (width 0.6) (layer B.Cu) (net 2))
 (segment (start 199.67 74) (end 164 74) (width 0.6) (layer B.Cu) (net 2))
 (segment (start 164 74) (end 155.56 82.44) (width 0.6) (layer B.Cu) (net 2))
 (segment (start 155.56 83.24) (end 154.059999 84.740001) (width 0.6) (layer B.Cu) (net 2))
 (segment (start 154.059999 84.740001) (end 140.840001 84.740001) (width 0.6) (layer B.Cu) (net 2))
 (segment (start 140.840001 84.740001) (end 140 83.9) (width 0.6) (layer B.Cu) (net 2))
 (segment (start 140 83.9) (end 140 82.5) (width 0.6) (layer B.Cu) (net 2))
 (segment (start 138.96 76.5) (end 138.96 59.736) (width 0.6) (layer B.Cu) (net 2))
 (segment (start 140 82.5) (end 140 81.1) (width 0.6) (layer B.Cu) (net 2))
 (segment (start 140 81.1) (end 138.96 80.06) (width 0.6) (layer B.Cu) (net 2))
 (segment (start 138.96 80.06) (end 138.96 78.85006) (width 0.6) (layer B.Cu) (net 2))
 (segment (start 138.96 78.85006) (end 138.96 76.5) (width 0.6) (layer B.Cu) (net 2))
 (segment (start 138.499999 84.000001) (end 140 82.5) (width 0.6) (layer B.Cu) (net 2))
 (segment (start 133.799999 84.000001) (end 138.499999 84.000001) (width 0.6) (layer B.Cu) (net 2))
 (segment (start 111.896841 84.000001) (end 133.799999 84.000001) (width 0.6) (layer B.Cu) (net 2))
 (segment (start 133.799999 84.000001) (end 135.3 82.5) (width 0.6) (layer B.Cu) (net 2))
 (segment (start 135.3 82.5) (end 135.5 82.5) (width 0.6) (layer B.Cu) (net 2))
 (segment (start 112 46.5) (end 107.5 51) (width 0.6) (layer B.Cu) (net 2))
 (segment (start 107.5 51) (end 107.5 54.5) (width 0.6) (layer B.Cu) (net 2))
 (segment (start 141.5 76.5) (end 141.5 74.14994) (width 0.6) (layer F.Cu) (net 5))
 (segment (start 141.5 74.14994) (end 139.35006 72) (width 0.6) (layer F.Cu) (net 5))
 (segment (start 127.25 65.25) (end 127.25 58.75) (width 0.6) (layer F.Cu) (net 5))
 (segment (start 139.35006 72) (end 134 72) (width 0.6) (layer F.Cu) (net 5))
 (segment (start 134 72) (end 127.25 65.25) (width 0.6) (layer F.Cu) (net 5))
 (segment (start 127.25 58.75) (end 121.75 53.25) (width 0.6) (layer F.Cu) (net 5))
 (segment (start 121.75 53.25) (end 119.25 53.25) (width 0.6) (layer F.Cu) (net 5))
 (segment (start 141.5 76.5) (end 142.94963 76.5) (width 0.6) (layer B.Cu) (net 5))
 (segment (start 142.94963 76.5) (end 144 77.55037) (width 0.6) (layer B.Cu) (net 5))
 (segment (start 144 77.55037) (end 144 81.1) (width 0.6) (layer B.Cu) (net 5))
 (segment (start 144 81.1) (end 144 82.5) (width 0.6) (layer B.Cu) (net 5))
 (segment (start 136.42 76.5) (end 136.42 78.85006) (width 0.6) (layer F.Cu) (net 6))
 (segment (start 136.42 78.85006) (end 140.18994 82.62) (width 0.6) (layer F.Cu) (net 6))
 (segment (start 140.18994 82.62) (end 153.02 82.62) (width 0.6) (layer F.Cu) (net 6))
 (segment (start 131.5 82.5) (end 131.7 82.5) (width 0.6) (layer B.Cu) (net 6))
 (segment (start 131.7 82.5) (end 136.42 77.78) (width 0.6) (layer B.Cu) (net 6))
 (segment (start 136.42 77.78) (end 136.42 76.5) (width 0.6) (layer B.Cu) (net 6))
 (segment (start 189.96 49.5) (end 189.96 50.50057) (width 0.25) (layer F.Cu) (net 7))
 (segment (start 189.96 50.50057) (end 192.45943 53) (width 0.25) (layer F.Cu) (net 7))
 (segment (start 195.5 53.5) (end 195.5 61.04) (width 0.25) (layer F.Cu) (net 7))
 (segment (start 192.45943 53) (end 195 53) (width 0.25) (layer F.Cu) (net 7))
 (segment (start 195 53) (end 195.5 53.5) (width 0.25) (layer F.Cu) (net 7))
 (segment (start 195.5 61.04) (end 194.799999 61.740001) (width 0.25) (layer F.Cu) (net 7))
 (segment (start 194.799999 61.740001) (end 194 62.54) (width 0.25) (layer F.Cu) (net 7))
 (segment (start 192.5 49.5) (end 196 49.5) (width 0.25) (layer B.Cu) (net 8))
 (segment (start 163.18 64.44) (end 163.18 67.38) (width 0.25) (layer F.Cu) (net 10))
 (segment (start 171.5 56.12) (end 163.18 64.44) (width 0.25) (layer F.Cu) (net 10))
 (segment (start 203 54.5) (end 203.761999 53.738001) (width 0.25) (layer B.Cu) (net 11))
 (segment (start 203.761999 53.738001) (end 203.761999 48.761999) (width 0.25) (layer B.Cu) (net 11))
 (segment (start 203.761999 48.761999) (end 201.5 46.5) (width 0.25) (layer B.Cu) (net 11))
 (segment (start 201.5 46.5) (end 181.5 46.5) (width 0.25) (layer B.Cu) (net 11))
 (segment (start 181.5 46.5) (end 174 54) (width 0.25) (layer B.Cu) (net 11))
 (segment (start 174 54) (end 170.5 54) (width 0.25) (layer B.Cu) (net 11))
 (segment (start 170.5 54) (end 168.96 55.54) (width 0.25) (layer B.Cu) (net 11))
 (segment (start 168.96 55.54) (end 168.96 56.12) (width 0.25) (layer B.Cu) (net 11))
 (segment (start 198.5 67) (end 197 65.5) (width 0.25) (layer B.Cu) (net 11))
 (segment (start 197 65.5) (end 186.5 65.5) (width 0.25) (layer B.Cu) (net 11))
 (segment (start 186.5 65.5) (end 180 59) (width 0.25) (layer B.Cu) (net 11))
 (segment (start 180 59) (end 171 59) (width 0.25) (layer B.Cu) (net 11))
 (segment (start 171 59) (end 169 57) (width 0.25) (layer B.Cu) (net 11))
 (segment (start 169 57) (end 169 56.16) (width 0.25) (layer B.Cu) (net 11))
 (segment (start 169 56.16) (end 168.96 56.12) (width 0.25) (layer B.Cu) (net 11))
 (segment (start 198.5 67) (end 198.5 71.5) (width 0.25) (layer B.Cu) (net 11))
 (segment (start 198.5 71.5) (end 199 72) (width 0.25) (layer B.Cu) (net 11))
 (segment (start 161.34 56.12) (end 161.34 63) (width 0.25) (layer B.Cu) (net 13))
 (segment (start 161.34 63) (end 165.72 67.38) (width 0.25) (layer B.Cu) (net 13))
 (segment (start 166.42 56.12) (end 166.42 60.46) (width 0.25) (layer B.Cu) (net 12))
 (segment (start 166.42 60.46) (end 173.34 67.38) (width 0.25) (layer B.Cu) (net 12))
 (segment (start 200 47.5) (end 200 49.5) (width 0.6) (layer B.Cu) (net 14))
 (segment (start 189.794541 47.254089) (end 199.754089 47.254089) (width 0.6) (layer F.Cu) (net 14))
 (segment (start 199.754089 47.254089) (end 200 47.5) (width 0.6) (layer F.Cu) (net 14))
 (via (at 200 47.5) (size 0.8) (drill 0.5) (layers F.Cu B.Cu) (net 14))
 (segment (start 170.8 67.38) (end 170.8 66.24863) (width 0.6) (layer F.Cu) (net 14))
 (segment (start 170.8 66.24863) (end 189.794541 47.254089) (width 0.6) (layer F.Cu) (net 14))
 (segment (start 110 80) (end 115 80) (width 0.6) (layer F.Cu) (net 1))
 (segment (start 115 80) (end 117.851499 77.148501) (width 0.6) (layer F.Cu) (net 1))
 (segment (start 119.25 50.75) (end 117.851499 52.148501) (width 0.6) (layer F.Cu) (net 1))
 (segment (start 117.851499 52.148501) (end 117.851499 77.148501) (width 0.6) (layer F.Cu) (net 1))
 (segment (start 175.88 67.38) (end 188.34 54.92) (width 0.25) (layer F.Cu) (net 15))
 (segment (start 188.34 54.92) (end 194 54.92) (width 0.25) (layer F.Cu) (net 15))
 (segment (start 178.42 67.38) (end 180.05 65.75) (width 0.25) (layer F.Cu) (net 16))
 (segment (start 180.05 65.75) (end 187.75 65.75) (width 0.25) (layer F.Cu) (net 16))
 (segment (start 191.75 61.75) (end 191.75 59.71) (width 0.25) (layer F.Cu) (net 16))
 (segment (start 187.75 65.75) (end 191.75 61.75) (width 0.25) (layer F.Cu) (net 16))
 (segment (start 191.75 59.71) (end 193.200001 58.259999) (width 0.25) (layer F.Cu) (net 16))
 (segment (start 193.200001 58.259999) (end 194 57.46) (width 0.25) (layer F.Cu) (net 16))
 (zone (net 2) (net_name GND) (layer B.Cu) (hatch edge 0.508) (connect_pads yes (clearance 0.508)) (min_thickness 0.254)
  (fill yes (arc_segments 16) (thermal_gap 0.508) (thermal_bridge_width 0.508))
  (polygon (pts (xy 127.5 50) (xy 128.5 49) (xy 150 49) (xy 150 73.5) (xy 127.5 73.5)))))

